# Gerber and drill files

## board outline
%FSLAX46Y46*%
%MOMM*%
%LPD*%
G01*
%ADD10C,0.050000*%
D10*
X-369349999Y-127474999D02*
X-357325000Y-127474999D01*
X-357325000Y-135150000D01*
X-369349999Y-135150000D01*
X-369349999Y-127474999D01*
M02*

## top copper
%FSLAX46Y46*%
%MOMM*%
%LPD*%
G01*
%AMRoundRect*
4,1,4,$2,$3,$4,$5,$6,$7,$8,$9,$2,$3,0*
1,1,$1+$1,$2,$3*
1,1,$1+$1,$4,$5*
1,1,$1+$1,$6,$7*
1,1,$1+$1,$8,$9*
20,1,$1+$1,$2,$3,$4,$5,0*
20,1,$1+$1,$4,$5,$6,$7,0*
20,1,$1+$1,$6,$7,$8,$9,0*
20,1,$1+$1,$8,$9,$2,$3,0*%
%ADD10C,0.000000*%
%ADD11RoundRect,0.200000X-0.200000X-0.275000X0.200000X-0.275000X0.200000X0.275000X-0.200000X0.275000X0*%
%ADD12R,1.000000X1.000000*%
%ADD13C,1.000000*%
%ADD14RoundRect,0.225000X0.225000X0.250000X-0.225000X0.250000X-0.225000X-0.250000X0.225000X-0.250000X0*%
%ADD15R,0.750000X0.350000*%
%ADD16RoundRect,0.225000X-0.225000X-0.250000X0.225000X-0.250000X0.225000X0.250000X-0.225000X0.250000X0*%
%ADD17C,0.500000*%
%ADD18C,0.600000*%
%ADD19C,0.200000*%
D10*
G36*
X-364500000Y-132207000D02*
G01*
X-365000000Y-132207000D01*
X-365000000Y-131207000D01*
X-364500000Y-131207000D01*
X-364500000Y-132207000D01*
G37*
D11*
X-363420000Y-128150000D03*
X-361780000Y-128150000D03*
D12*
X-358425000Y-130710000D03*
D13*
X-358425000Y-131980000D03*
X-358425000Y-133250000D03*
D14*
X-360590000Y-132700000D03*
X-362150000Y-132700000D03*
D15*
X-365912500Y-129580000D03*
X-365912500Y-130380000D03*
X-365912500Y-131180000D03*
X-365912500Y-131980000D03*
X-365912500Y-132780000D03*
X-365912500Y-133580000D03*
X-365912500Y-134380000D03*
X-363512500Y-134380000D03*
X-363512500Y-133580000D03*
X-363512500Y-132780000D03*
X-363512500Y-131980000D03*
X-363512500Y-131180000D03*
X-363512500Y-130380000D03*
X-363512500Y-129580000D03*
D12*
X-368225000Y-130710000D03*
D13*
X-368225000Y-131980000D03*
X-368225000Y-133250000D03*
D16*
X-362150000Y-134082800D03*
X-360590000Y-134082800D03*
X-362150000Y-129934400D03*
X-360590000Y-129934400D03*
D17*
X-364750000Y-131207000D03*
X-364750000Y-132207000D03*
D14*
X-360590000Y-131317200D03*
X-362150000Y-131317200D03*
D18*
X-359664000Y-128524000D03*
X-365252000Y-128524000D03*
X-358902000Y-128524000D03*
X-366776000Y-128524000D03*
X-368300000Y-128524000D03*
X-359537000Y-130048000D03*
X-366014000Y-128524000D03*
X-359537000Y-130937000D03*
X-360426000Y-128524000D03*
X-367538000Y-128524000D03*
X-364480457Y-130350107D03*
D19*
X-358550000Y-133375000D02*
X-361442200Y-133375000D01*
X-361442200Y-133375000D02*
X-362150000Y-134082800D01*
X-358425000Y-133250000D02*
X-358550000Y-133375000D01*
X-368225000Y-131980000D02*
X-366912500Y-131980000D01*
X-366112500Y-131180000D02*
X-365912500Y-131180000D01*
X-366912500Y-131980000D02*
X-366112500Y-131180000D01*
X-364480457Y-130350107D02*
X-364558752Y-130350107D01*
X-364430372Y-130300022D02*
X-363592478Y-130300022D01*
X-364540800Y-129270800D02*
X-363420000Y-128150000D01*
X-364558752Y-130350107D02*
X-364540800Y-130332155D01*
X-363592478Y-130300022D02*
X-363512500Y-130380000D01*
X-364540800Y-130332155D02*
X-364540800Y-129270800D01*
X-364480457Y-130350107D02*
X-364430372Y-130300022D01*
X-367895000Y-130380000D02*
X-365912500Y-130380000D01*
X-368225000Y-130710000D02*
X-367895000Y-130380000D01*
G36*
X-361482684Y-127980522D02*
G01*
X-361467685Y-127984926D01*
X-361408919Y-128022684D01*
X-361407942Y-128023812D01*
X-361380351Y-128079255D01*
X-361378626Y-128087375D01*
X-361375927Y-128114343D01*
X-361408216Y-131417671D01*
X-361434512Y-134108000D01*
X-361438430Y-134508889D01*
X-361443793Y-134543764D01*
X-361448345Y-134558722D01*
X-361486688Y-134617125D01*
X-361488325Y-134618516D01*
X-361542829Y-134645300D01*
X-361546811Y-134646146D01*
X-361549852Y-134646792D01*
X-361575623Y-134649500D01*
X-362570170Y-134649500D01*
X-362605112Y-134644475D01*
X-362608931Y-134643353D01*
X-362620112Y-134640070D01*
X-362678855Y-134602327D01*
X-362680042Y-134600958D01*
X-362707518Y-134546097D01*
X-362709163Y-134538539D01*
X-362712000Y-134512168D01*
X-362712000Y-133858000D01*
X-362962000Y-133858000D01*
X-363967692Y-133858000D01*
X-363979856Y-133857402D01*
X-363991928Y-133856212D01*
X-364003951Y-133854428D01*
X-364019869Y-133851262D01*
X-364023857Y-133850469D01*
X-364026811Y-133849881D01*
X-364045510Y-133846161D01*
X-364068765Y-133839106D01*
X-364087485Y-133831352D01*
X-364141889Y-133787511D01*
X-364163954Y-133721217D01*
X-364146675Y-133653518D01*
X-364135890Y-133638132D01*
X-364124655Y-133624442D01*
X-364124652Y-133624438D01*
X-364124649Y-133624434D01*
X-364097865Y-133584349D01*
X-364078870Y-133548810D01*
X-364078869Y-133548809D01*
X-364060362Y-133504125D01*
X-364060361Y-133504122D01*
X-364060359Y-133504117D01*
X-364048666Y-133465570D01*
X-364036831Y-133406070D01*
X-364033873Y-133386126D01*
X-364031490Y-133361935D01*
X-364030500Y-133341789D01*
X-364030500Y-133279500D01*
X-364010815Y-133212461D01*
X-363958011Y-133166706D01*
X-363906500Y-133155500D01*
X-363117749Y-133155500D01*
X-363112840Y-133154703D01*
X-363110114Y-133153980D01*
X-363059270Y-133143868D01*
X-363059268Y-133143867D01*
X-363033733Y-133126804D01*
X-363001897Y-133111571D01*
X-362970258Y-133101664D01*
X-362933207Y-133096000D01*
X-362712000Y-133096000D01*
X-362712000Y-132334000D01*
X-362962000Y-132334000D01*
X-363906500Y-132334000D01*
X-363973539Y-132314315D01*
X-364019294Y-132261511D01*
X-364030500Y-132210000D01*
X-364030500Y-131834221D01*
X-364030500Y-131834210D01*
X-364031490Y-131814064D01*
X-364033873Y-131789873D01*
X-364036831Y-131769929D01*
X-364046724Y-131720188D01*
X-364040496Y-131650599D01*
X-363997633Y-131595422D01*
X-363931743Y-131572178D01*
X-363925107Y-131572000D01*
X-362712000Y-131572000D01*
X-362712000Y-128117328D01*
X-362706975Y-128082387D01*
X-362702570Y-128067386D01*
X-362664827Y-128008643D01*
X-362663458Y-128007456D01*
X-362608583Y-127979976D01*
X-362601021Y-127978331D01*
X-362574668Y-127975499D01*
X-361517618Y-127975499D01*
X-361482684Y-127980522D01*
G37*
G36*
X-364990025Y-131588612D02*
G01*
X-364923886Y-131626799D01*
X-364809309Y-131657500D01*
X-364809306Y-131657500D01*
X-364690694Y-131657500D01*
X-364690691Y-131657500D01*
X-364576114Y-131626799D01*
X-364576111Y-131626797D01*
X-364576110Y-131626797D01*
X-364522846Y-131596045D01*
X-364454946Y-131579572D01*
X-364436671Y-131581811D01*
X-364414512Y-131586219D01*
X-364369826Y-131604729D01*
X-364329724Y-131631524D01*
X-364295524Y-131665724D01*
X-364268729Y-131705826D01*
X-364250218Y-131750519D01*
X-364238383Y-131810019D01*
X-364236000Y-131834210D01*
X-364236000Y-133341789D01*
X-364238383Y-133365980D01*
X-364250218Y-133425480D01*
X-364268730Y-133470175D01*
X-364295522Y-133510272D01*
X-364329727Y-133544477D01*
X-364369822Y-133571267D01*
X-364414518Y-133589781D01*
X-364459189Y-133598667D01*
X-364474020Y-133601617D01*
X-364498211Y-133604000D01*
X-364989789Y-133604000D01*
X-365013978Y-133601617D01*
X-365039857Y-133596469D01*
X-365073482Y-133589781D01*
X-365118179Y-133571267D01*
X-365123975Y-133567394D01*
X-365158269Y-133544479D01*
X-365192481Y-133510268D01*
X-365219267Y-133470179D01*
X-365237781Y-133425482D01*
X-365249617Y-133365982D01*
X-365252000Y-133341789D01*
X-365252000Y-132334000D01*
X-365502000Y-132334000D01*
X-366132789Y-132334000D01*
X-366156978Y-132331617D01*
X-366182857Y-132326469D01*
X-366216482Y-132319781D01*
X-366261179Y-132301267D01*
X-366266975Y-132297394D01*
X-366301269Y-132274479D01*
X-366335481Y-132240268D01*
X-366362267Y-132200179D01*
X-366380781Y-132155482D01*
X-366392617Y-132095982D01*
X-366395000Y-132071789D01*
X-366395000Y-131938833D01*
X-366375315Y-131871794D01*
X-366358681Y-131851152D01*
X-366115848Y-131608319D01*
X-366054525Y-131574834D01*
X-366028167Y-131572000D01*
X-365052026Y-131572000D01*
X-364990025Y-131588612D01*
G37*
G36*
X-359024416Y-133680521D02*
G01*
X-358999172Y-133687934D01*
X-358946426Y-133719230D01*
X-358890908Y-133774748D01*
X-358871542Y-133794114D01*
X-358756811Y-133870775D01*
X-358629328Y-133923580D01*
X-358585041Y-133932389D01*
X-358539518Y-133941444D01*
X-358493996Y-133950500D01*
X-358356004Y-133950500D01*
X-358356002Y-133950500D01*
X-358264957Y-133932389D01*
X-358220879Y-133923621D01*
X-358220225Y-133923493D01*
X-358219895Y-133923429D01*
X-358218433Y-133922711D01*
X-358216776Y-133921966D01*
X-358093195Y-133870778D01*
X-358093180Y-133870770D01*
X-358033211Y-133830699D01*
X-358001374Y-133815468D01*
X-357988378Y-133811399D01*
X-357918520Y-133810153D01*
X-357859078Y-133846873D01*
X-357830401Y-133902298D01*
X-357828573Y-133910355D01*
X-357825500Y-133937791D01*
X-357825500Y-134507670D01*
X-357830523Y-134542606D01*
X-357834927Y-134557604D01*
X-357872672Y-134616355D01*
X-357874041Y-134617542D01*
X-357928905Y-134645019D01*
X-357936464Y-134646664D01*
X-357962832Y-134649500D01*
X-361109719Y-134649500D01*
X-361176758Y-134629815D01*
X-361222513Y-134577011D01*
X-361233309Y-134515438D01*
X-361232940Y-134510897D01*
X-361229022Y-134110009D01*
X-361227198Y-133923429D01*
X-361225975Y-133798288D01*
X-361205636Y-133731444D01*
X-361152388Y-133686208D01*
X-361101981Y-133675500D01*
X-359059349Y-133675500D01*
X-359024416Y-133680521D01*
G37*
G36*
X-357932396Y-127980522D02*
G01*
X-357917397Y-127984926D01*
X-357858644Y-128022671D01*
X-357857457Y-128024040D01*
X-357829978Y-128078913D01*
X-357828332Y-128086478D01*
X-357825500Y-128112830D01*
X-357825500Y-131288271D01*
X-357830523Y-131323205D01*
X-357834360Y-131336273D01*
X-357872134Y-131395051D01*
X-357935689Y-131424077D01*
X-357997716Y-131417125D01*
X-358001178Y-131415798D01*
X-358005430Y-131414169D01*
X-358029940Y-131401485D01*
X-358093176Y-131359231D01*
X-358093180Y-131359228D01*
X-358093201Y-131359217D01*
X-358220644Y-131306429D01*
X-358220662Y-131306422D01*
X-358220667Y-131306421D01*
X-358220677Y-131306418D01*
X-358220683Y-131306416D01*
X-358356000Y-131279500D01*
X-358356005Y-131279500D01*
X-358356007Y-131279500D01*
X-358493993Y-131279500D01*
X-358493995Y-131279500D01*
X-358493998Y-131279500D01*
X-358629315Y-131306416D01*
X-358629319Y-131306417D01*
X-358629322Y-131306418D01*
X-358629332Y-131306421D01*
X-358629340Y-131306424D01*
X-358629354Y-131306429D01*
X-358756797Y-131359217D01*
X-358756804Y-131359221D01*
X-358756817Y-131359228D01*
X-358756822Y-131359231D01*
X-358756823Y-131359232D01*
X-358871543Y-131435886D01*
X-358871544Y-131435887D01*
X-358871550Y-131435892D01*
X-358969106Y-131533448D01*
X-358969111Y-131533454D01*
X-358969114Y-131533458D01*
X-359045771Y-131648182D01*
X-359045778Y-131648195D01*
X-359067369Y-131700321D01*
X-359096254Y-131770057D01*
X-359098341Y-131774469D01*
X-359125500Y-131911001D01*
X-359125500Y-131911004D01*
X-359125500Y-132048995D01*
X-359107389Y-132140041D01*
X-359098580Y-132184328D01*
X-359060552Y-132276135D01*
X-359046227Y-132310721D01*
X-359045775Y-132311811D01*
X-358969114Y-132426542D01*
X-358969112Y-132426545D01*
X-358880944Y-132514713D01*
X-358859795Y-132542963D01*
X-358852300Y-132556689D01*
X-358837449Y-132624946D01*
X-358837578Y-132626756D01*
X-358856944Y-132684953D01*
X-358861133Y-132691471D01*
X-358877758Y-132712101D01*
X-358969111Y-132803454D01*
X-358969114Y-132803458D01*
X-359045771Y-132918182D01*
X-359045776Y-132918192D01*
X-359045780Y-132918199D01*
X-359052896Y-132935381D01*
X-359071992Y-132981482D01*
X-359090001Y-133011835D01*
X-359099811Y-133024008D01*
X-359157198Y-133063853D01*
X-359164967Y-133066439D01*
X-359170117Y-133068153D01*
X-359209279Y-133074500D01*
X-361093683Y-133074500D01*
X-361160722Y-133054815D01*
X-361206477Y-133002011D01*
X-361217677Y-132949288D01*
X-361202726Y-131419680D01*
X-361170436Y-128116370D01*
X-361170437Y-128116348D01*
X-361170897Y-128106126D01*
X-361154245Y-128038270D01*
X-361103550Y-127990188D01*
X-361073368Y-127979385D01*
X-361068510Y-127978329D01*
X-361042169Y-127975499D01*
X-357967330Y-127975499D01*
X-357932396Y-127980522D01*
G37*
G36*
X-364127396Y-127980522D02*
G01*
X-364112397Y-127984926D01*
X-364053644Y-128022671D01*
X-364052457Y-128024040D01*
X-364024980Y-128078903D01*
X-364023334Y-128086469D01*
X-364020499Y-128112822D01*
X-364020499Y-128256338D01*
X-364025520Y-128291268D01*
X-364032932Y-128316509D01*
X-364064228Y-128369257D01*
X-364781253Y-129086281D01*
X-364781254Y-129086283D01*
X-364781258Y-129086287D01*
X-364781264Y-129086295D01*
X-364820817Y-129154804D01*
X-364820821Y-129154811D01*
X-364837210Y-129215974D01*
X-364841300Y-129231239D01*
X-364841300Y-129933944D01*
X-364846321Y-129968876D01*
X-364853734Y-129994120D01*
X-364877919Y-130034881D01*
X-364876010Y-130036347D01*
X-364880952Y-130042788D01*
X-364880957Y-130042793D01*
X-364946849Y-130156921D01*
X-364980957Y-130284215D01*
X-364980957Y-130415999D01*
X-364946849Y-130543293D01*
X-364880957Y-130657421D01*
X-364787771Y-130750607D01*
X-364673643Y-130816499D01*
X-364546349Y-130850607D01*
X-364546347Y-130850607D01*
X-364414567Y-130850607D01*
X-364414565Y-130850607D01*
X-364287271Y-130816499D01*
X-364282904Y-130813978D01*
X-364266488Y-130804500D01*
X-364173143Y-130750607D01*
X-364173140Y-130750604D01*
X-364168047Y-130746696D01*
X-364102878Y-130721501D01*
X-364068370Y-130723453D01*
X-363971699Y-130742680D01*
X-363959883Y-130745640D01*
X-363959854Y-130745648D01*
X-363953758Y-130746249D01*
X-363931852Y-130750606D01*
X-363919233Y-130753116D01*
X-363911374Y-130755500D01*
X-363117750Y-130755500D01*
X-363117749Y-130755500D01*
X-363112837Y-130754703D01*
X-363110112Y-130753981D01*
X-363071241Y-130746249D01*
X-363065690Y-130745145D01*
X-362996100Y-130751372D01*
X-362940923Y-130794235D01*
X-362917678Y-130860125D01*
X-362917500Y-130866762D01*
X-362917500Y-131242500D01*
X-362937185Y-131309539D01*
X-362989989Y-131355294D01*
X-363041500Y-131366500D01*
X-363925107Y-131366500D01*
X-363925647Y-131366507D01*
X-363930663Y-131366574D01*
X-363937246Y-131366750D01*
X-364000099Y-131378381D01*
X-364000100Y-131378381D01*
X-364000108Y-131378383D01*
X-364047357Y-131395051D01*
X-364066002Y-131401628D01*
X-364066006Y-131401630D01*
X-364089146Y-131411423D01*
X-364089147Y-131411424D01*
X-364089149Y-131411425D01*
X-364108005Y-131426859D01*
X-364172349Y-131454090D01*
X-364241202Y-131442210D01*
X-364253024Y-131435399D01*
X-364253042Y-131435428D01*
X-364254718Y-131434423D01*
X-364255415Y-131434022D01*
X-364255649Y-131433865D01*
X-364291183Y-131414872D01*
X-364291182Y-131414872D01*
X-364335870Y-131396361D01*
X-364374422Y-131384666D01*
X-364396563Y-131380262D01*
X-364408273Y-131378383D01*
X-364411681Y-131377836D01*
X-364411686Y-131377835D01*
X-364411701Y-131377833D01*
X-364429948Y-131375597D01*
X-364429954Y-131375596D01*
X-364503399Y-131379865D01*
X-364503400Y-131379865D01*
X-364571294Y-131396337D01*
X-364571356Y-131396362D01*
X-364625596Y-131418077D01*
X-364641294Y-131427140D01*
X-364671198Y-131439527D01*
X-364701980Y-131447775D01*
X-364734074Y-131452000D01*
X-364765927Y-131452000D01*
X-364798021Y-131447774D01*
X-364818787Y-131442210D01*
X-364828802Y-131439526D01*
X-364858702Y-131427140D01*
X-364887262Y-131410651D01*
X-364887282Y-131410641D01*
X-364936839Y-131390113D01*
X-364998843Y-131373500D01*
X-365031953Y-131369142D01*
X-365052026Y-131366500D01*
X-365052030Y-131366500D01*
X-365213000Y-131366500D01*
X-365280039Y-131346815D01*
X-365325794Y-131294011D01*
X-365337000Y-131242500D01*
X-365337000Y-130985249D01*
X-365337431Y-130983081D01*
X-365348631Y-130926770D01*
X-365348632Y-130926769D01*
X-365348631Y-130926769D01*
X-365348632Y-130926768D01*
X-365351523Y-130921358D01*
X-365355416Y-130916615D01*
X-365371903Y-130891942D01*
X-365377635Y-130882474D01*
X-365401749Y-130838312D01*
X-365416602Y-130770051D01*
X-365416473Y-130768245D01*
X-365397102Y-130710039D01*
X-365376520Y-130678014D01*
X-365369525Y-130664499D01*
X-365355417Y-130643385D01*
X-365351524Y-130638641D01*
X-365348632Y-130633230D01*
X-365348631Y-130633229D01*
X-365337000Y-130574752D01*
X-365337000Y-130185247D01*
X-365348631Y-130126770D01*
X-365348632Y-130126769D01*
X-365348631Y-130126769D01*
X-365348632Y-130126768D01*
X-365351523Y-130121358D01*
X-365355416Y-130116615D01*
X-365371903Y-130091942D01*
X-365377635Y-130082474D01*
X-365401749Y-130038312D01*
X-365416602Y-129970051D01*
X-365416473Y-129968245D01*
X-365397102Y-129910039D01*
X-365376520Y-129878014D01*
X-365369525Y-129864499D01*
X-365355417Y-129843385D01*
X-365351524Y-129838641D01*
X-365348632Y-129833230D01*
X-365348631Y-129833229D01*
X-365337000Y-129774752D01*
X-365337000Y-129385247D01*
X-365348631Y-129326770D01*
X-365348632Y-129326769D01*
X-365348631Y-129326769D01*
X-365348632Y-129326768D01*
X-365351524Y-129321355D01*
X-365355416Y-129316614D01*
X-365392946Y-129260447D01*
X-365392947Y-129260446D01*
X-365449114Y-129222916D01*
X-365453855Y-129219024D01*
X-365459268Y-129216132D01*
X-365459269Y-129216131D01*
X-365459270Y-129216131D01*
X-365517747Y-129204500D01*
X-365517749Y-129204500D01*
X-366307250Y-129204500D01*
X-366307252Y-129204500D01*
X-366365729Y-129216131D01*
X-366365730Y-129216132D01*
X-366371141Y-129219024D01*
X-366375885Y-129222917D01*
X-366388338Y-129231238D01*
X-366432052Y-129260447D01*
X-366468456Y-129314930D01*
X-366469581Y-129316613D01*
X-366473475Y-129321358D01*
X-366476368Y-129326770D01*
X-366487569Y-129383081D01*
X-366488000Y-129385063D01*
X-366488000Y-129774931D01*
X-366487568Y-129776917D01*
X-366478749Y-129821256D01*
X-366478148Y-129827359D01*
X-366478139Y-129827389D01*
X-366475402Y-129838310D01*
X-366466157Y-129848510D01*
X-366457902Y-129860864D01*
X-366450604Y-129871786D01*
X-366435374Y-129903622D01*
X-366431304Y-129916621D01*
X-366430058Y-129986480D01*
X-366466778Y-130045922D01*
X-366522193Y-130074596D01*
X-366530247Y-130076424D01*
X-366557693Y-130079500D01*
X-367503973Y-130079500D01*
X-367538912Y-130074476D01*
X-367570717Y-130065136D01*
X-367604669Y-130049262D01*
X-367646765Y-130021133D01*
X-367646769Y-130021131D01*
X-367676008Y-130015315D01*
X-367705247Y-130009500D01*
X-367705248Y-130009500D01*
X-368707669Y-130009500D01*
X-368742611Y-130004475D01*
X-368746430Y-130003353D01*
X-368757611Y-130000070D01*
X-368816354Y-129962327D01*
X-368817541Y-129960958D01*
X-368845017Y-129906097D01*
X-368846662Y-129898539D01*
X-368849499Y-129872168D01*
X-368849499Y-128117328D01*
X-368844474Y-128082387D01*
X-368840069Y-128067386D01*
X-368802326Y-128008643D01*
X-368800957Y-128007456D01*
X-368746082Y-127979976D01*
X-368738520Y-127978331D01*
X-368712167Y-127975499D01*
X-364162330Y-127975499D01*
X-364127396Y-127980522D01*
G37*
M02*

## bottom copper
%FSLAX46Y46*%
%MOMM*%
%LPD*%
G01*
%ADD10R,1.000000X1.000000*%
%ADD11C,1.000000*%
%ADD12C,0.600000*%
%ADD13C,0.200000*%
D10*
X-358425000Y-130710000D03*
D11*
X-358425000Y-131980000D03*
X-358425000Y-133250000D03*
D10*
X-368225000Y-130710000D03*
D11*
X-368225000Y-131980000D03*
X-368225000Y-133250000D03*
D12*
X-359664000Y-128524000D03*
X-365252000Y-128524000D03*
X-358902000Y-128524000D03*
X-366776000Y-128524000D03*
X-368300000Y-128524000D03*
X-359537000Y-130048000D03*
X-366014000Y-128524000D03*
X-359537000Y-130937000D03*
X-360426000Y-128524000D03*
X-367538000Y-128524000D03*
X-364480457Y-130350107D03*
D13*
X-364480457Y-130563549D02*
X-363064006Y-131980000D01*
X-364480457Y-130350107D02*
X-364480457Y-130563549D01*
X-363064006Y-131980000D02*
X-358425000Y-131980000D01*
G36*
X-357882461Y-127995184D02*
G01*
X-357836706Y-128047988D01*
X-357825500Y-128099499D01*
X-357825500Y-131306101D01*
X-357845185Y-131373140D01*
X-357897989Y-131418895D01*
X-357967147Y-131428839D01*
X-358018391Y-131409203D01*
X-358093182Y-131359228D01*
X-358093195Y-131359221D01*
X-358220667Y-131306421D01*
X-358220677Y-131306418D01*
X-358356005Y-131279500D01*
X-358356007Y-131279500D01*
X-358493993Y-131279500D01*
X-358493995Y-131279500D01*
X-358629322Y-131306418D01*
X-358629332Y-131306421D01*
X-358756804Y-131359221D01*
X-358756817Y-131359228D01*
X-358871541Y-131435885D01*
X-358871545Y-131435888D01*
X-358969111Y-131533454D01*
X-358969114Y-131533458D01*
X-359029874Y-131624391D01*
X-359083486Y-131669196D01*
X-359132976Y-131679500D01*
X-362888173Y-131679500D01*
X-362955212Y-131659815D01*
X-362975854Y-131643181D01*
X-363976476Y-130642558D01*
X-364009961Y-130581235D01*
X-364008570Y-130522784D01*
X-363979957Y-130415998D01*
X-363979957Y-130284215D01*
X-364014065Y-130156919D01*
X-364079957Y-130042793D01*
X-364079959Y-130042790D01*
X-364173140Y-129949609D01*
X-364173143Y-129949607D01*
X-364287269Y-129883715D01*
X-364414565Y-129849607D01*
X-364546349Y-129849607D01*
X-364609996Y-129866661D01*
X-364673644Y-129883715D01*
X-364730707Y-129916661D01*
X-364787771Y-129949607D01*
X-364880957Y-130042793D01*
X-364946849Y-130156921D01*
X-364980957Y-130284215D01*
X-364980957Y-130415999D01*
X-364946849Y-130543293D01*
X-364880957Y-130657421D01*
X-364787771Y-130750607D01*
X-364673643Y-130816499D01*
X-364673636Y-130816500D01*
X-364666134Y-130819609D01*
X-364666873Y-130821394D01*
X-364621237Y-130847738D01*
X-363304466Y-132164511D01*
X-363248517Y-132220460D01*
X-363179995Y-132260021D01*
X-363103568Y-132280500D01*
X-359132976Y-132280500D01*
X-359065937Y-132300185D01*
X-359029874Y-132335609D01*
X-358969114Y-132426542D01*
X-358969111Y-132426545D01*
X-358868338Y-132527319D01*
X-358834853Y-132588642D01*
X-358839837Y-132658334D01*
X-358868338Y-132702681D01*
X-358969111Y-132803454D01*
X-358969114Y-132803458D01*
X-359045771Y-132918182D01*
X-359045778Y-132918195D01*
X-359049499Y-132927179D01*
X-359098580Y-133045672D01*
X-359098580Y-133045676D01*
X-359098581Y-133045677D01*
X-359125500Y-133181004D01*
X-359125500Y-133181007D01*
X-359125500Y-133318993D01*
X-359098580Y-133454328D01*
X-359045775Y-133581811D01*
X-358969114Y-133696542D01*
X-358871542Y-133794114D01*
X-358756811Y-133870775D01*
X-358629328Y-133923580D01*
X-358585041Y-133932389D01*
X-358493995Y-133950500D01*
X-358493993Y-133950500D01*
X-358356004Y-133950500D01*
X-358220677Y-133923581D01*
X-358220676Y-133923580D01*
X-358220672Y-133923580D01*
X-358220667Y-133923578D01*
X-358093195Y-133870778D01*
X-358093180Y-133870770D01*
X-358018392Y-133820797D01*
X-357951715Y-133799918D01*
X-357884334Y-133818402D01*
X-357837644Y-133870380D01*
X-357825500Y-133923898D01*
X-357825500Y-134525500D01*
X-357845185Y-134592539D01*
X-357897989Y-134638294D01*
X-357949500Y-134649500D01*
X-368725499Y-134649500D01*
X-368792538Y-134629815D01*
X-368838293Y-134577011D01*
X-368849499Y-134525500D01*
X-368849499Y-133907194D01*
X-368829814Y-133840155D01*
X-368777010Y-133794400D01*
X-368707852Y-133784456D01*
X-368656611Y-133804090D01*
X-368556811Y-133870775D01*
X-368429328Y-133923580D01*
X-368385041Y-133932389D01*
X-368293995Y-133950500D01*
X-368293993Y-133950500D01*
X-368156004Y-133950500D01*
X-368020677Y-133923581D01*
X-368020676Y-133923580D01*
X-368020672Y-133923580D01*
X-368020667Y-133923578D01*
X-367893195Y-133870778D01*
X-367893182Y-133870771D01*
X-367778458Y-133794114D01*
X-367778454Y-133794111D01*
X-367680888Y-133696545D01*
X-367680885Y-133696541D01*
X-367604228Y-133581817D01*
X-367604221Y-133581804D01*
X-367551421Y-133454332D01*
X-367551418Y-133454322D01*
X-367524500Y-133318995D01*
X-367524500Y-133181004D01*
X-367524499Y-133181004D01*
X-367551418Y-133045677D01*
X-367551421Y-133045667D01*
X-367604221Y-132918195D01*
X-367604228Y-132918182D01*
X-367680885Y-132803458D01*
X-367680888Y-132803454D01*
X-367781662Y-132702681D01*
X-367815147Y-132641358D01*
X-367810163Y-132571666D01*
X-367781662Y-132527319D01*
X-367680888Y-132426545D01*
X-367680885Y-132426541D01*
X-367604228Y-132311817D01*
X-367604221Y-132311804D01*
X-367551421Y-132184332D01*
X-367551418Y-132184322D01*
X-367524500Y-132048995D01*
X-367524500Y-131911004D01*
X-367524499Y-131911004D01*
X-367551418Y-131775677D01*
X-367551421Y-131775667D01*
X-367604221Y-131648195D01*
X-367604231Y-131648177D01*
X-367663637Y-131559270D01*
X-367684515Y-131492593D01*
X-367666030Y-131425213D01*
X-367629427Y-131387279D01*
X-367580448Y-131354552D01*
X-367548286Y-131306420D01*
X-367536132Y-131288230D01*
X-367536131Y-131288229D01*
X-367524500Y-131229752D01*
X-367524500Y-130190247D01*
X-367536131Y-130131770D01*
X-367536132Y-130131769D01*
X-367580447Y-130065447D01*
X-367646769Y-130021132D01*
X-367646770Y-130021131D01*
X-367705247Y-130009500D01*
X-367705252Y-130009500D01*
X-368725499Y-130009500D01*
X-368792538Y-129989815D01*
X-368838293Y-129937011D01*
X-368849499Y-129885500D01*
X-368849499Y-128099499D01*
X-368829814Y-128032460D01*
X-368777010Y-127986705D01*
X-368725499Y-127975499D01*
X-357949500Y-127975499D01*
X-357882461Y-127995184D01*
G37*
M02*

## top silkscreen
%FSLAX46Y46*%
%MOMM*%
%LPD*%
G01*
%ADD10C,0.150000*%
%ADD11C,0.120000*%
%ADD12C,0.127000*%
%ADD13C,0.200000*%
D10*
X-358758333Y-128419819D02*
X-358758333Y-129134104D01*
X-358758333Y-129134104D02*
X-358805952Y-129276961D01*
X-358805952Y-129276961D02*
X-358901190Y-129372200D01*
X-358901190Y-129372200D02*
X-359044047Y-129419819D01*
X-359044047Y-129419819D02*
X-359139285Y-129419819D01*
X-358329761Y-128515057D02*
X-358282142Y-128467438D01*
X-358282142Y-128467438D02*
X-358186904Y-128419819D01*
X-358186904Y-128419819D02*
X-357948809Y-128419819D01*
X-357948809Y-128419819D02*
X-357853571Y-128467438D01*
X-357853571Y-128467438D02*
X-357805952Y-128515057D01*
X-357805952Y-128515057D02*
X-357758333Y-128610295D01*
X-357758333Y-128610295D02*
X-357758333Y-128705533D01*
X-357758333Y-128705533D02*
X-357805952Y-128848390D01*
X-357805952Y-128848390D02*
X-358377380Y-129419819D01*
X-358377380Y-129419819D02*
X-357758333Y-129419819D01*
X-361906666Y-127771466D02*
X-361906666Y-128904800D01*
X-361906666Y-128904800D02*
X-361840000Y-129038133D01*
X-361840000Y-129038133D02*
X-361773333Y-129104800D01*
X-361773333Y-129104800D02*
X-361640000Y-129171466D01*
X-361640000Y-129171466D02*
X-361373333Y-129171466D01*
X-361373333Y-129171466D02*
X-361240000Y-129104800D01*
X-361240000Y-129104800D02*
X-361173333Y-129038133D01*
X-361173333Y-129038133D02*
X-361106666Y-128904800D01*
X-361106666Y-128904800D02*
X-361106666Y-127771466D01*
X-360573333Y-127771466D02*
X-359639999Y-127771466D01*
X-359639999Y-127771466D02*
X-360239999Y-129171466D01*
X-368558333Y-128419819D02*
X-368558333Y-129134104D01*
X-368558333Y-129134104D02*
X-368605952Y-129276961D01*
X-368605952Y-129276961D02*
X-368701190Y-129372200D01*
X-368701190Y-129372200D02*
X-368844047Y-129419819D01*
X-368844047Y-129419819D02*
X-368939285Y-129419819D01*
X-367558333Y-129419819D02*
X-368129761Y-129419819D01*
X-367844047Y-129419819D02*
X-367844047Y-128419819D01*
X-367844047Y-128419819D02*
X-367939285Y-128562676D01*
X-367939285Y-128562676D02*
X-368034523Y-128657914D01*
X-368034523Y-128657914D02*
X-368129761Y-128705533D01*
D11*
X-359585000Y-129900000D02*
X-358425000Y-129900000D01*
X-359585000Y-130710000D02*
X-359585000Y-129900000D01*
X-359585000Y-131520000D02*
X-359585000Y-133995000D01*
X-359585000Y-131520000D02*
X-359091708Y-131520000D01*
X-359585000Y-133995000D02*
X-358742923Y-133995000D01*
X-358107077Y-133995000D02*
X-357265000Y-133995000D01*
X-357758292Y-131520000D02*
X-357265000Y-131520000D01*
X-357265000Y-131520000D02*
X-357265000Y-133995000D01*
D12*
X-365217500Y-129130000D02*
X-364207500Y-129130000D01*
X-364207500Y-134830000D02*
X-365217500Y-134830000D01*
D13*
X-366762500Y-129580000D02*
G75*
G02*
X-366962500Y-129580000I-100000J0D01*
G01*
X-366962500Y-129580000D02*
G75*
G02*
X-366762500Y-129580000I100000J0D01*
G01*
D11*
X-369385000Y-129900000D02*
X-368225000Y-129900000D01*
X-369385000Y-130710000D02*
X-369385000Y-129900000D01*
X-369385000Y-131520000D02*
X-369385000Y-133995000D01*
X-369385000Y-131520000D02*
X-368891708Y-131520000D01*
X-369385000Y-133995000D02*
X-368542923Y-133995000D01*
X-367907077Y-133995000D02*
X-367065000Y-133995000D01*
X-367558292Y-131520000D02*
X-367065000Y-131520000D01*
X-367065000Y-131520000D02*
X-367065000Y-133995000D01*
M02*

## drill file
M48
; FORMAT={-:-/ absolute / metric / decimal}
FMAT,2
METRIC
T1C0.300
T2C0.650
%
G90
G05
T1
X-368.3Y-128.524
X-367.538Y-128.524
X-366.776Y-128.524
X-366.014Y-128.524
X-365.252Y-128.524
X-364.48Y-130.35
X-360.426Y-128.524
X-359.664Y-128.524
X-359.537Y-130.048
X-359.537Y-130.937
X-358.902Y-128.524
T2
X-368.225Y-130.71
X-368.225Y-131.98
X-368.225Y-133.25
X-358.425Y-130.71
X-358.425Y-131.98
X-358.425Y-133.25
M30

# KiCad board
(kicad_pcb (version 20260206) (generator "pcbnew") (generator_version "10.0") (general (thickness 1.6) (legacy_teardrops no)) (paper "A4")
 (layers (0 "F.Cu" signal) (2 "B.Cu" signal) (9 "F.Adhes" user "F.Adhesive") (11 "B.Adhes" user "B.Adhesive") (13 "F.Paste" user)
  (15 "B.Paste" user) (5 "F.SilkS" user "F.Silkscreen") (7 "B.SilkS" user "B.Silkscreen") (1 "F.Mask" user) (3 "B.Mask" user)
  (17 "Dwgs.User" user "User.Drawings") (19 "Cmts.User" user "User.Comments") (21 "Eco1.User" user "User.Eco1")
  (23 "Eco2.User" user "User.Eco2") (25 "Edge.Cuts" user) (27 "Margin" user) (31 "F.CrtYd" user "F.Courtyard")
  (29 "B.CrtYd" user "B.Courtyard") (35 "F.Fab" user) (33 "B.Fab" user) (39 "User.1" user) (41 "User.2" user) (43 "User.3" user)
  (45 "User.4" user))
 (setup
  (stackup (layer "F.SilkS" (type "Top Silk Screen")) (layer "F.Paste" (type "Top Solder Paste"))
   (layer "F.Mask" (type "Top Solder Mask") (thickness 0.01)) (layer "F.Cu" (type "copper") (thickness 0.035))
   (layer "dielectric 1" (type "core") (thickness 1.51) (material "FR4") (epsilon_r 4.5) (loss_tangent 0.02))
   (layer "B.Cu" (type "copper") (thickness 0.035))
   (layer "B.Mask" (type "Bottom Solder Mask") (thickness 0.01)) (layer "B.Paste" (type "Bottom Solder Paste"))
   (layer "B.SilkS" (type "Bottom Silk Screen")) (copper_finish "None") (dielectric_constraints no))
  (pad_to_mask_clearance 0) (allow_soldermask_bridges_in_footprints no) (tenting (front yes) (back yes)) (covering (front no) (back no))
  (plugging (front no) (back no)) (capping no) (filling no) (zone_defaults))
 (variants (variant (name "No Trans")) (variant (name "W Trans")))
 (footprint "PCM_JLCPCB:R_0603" (layer "F.Cu") (at -362.6 128.15)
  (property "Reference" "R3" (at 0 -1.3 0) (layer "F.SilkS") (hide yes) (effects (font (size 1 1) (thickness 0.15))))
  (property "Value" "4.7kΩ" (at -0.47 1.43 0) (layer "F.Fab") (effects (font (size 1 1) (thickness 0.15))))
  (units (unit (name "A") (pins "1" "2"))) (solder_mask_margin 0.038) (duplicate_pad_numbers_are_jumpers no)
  (pad "1" smd roundrect (at -0.82 0) (size 0.8 0.95) (layers "F.Cu" "F.Mask" "F.Paste") (roundrect_rratio 0.25) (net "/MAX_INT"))
  (pad "2" smd roundrect (at 0.82 0) (size 0.8 0.95) (layers "F.Cu" "F.Mask" "F.Paste") (roundrect_rratio 0.25) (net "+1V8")))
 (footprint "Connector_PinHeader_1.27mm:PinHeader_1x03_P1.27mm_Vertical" (layer "F.Cu") (at -358.425 130.71)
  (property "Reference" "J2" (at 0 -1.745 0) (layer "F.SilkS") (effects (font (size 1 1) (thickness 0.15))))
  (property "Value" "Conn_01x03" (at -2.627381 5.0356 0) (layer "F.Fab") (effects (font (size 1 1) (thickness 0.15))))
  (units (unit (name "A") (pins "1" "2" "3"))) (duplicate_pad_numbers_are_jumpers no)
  (fp_line (start -1.16 -0.81) (end 0 -0.81) (stroke (width 0.12) (type solid)) (layer "F.SilkS"))
  (fp_line (start -1.16 0) (end -1.16 -0.81) (stroke (width 0.12) (type solid)) (layer "F.SilkS"))
  (fp_line (start -1.16 0.81) (end -1.16 3.285) (stroke (width 0.12) (type solid)) (layer "F.SilkS"))
  (fp_line (start -1.16 0.81) (end -0.666708 0.81) (stroke (width 0.12) (type solid)) (layer "F.SilkS"))
  (fp_line (start -1.16 3.285) (end -0.317923 3.285) (stroke (width 0.12) (type solid)) (layer "F.SilkS"))
  (fp_line (start 0.317923 3.285) (end 1.16 3.285) (stroke (width 0.12) (type solid)) (layer "F.SilkS"))
  (fp_line (start 0.666708 0.81) (end 1.16 0.81) (stroke (width 0.12) (type solid)) (layer "F.SilkS"))
  (fp_line (start 1.16 0.81) (end 1.16 3.285) (stroke (width 0.12) (type solid)) (layer "F.SilkS"))
  (pad "1" thru_hole rect (at 0 0) (size 1 1) (drill 0.65) (layers "*.Cu" "*.Mask") (remove_unused_layers no) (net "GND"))
  (pad "2" thru_hole circle (at 0 1.27) (size 1 1) (drill 0.65) (layers "*.Cu" "*.Mask") (remove_unused_layers no) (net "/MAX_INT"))
  (pad "3" thru_hole circle (at 0 2.54) (size 1 1) (drill 0.65) (layers "*.Cu" "*.Mask") (remove_unused_layers no) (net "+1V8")))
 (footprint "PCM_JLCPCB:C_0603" (layer "F.Cu") (at -361.37 132.7 180)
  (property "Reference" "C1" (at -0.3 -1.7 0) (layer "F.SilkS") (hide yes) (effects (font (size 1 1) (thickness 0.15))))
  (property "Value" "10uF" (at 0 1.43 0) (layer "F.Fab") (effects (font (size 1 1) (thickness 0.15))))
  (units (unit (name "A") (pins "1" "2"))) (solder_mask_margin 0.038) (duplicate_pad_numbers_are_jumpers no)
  (pad "1" smd roundrect (at -0.78 0 180) (size 0.9 0.95) (layers "F.Cu" "F.Mask" "F.Paste") (roundrect_rratio 0.25) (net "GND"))
  (pad "2" smd roundrect (at 0.78 0 180) (size 0.9 0.95) (layers "F.Cu" "F.Mask" "F.Paste") (roundrect_rratio 0.25) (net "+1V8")))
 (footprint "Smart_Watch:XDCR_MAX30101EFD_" (layer "F.Cu") (at -364.7125 131.98)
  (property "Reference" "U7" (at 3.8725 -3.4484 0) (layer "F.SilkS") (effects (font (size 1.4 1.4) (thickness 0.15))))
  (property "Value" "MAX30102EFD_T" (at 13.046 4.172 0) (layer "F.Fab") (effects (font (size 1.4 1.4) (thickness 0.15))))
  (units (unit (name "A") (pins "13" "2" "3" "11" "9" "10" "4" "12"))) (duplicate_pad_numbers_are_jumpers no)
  (fp_line (start -0.505 -2.85) (end 0.505 -2.85) (stroke (width 0.127) (type solid)) (layer "F.SilkS"))
  (fp_line (start 0.505 2.85) (end -0.505 2.85) (stroke (width 0.127) (type solid)) (layer "F.SilkS"))
  (fp_circle (center -2.15 -2.4) (end -2.05 -2.4) (stroke (width 0.2) (type solid)) (fill no) (layer "F.SilkS"))
  (pad "1" smd rect (at -1.2 -2.4) (size 0.75 0.35) (layers "F.Cu" "F.Mask" "F.Paste") (solder_mask_margin 0.102))
  (pad "2" smd rect (at -1.2 -1.6) (size 0.75 0.35) (layers "F.Cu" "F.Mask" "F.Paste") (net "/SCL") (solder_mask_margin 0.102))
  (pad "3" smd rect (at -1.2 -0.8) (size 0.75 0.35) (layers "F.Cu" "F.Mask" "F.Paste") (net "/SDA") (solder_mask_margin 0.102))
  (pad "4" smd rect (at -1.2 0) (size 0.75 0.35) (layers "F.Cu" "F.Mask" "F.Paste") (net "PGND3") (solder_mask_margin 0.102))
  (pad "5" smd rect (at -1.2 0.8) (size 0.75 0.35) (layers "F.Cu" "F.Mask" "F.Paste") (solder_mask_margin 0.102))
  (pad "6" smd rect (at -1.2 1.6) (size 0.75 0.35) (layers "F.Cu" "F.Mask" "F.Paste") (solder_mask_margin 0.102))
  (pad "7" smd rect (at -1.2 2.4) (size 0.75 0.35) (layers "F.Cu" "F.Mask" "F.Paste") (solder_mask_margin 0.102))
  (pad "8" smd rect (at 1.2 2.4) (size 0.75 0.35) (layers "F.Cu" "F.Mask" "F.Paste") (solder_mask_margin 0.102))
  (pad "9" smd rect (at 1.2 1.6) (size 0.75 0.35) (layers "F.Cu" "F.Mask" "F.Paste") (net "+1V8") (solder_mask_margin 0.102))
  (pad "10" smd rect (at 1.2 0.8) (size 0.75 0.35) (layers "F.Cu" "F.Mask" "F.Paste") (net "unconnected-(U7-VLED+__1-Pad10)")
   (solder_mask_margin 0.102))
  (pad "11" smd rect (at 1.2 0) (size 0.75 0.35) (layers "F.Cu" "F.Mask" "F.Paste") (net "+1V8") (solder_mask_margin 0.102))
  (pad "12" smd rect (at 1.2 -0.8) (size 0.75 0.35) (layers "F.Cu" "F.Mask" "F.Paste") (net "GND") (solder_mask_margin 0.102))
  (pad "13" smd rect (at 1.2 -1.6) (size 0.75 0.35) (layers "F.Cu" "F.Mask" "F.Paste") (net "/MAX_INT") (solder_mask_margin 0.102))
  (pad "14" smd rect (at 1.2 -2.4) (size 0.75 0.35) (layers "F.Cu" "F.Mask" "F.Paste") (solder_mask_margin 0.102)))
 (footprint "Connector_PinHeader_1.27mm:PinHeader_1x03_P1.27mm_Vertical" (layer "F.Cu") (at -368.225 130.71)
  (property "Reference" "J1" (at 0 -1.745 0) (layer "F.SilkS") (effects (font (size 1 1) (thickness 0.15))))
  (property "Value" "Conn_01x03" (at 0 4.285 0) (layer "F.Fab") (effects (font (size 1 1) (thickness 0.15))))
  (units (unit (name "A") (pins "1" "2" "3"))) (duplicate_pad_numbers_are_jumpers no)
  (fp_line (start -1.16 -0.81) (end 0 -0.81) (stroke (width 0.12) (type solid)) (layer "F.SilkS"))
  (fp_line (start -1.16 0) (end -1.16 -0.81) (stroke (width 0.12) (type solid)) (layer "F.SilkS"))
  (fp_line (start -1.16 0.81) (end -1.16 3.285) (stroke (width 0.12) (type solid)) (layer "F.SilkS"))
  (fp_line (start -1.16 0.81) (end -0.666708 0.81) (stroke (width 0.12) (type solid)) (layer "F.SilkS"))
  (fp_line (start -1.16 3.285) (end -0.317923 3.285) (stroke (width 0.12) (type solid)) (layer "F.SilkS"))
  (fp_line (start 0.317923 3.285) (end 1.16 3.285) (stroke (width 0.12) (type solid)) (layer "F.SilkS"))
  (fp_line (start 0.666708 0.81) (end 1.16 0.81) (stroke (width 0.12) (type solid)) (layer "F.SilkS"))
  (fp_line (start 1.16 0.81) (end 1.16 3.285) (stroke (width 0.12) (type solid)) (layer "F.SilkS"))
  (pad "1" thru_hole rect (at 0 0) (size 1 1) (drill 0.65) (layers "*.Cu" "*.Mask") (remove_unused_layers no) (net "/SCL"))
  (pad "2" thru_hole circle (at 0 1.27) (size 1 1) (drill 0.65) (layers "*.Cu" "*.Mask") (remove_unused_layers no) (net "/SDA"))
  (pad "3" thru_hole circle (at 0 2.54) (size 1 1) (drill 0.65) (layers "*.Cu" "*.Mask") (remove_unused_layers no)
   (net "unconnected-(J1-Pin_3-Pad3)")))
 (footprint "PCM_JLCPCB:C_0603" (layer "F.Cu") (at -361.37 134.0828)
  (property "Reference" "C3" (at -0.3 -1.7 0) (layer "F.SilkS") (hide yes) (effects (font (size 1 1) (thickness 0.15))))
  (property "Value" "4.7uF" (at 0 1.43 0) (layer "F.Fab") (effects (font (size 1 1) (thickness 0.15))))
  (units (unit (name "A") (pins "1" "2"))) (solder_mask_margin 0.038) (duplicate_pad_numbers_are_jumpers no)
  (pad "1" smd roundrect (at -0.78 0) (size 0.9 0.95) (layers "F.Cu" "F.Mask" "F.Paste") (roundrect_rratio 0.25) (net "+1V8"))
  (pad "2" smd roundrect (at 0.78 0) (size 0.9 0.95) (layers "F.Cu" "F.Mask" "F.Paste") (roundrect_rratio 0.25) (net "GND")))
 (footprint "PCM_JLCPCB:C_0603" (layer "F.Cu") (at -361.37 129.9344)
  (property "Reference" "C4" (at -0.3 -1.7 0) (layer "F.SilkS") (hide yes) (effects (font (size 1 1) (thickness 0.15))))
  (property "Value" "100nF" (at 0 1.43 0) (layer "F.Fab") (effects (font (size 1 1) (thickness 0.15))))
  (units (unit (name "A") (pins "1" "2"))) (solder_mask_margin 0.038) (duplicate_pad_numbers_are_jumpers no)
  (pad "1" smd roundrect (at -0.78 0) (size 0.9 0.95) (layers "F.Cu" "F.Mask" "F.Paste") (roundrect_rratio 0.25) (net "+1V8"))
  (pad "2" smd roundrect (at 0.78 0) (size 0.9 0.95) (layers "F.Cu" "F.Mask" "F.Paste") (roundrect_rratio 0.25) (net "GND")))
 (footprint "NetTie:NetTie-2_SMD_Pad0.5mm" (layer "F.Cu") (at -364.75 131.707 -90)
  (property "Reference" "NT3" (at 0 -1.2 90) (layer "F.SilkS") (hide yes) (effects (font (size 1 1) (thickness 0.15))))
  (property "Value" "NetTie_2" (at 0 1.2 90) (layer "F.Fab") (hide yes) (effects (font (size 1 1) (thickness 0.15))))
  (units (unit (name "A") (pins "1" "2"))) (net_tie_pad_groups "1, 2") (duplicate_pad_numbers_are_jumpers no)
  (fp_poly (pts (xy -0.5 -0.25) (xy 0.5 -0.25) (xy 0.5 0.25) (xy -0.5 0.25)) (stroke (width 0) (type solid)) (fill yes) (layer "F.Cu"))
  (pad "1" smd circle (at -0.5 0 270) (size 0.5 0.5) (layers "F.Cu") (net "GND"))
  (pad "2" smd circle (at 0.5 0 270) (size 0.5 0.5) (layers "F.Cu") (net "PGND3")))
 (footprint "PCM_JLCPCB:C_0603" (layer "F.Cu") (at -361.37 131.3172 180)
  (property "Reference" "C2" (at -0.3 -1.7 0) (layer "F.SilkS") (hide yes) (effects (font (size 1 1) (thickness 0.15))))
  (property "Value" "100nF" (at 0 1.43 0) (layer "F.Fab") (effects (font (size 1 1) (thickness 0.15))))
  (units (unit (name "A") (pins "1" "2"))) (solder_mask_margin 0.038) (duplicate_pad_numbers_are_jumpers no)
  (pad "1" smd roundrect (at -0.78 0 180) (size 0.9 0.95) (layers "F.Cu" "F.Mask" "F.Paste") (roundrect_rratio 0.25) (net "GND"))
  (pad "2" smd roundrect (at 0.78 0 180) (size 0.9 0.95) (layers "F.Cu" "F.Mask" "F.Paste") (roundrect_rratio 0.25) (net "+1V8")))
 (gr_rect (start -369.349999 127.474999) (end -357.325 135.15) (stroke (width 0.05) (type default)) (fill no) (layer "Edge.Cuts"))
 (via (at -359.664 128.524) (size 0.6) (drill 0.3) (layers "F.Cu" "B.Cu") (free yes) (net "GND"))
 (via (at -365.252 128.524) (size 0.6) (drill 0.3) (layers "F.Cu" "B.Cu") (free yes) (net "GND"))
 (via (at -358.902 128.524) (size 0.6) (drill 0.3) (layers "F.Cu" "B.Cu") (free yes) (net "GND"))
 (via (at -366.776 128.524) (size 0.6) (drill 0.3) (layers "F.Cu" "B.Cu") (free yes) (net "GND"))
 (via (at -368.3 128.524) (size 0.6) (drill 0.3) (layers "F.Cu" "B.Cu") (free yes) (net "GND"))
 (via (at -359.537 130.048) (size 0.6) (drill 0.3) (layers "F.Cu" "B.Cu") (free yes) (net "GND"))
 (via (at -366.014 128.524) (size 0.6) (drill 0.3) (layers "F.Cu" "B.Cu") (free yes) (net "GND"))
 (via (at -359.537 130.937) (size 0.6) (drill 0.3) (layers "F.Cu" "B.Cu") (free yes) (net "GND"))
 (via (at -360.426 128.524) (size 0.6) (drill 0.3) (layers "F.Cu" "B.Cu") (free yes) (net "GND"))
 (via (at -367.538 128.524) (size 0.6) (drill 0.3) (layers "F.Cu" "B.Cu") (free yes) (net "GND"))
 (segment (start -358.55 133.375) (end -361.4422 133.375) (width 0.2) (layer "F.Cu") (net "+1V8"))
 (segment (start -361.4422 133.375) (end -362.15 134.0828) (width 0.2) (layer "F.Cu") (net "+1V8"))
 (segment (start -358.425 133.25) (end -358.55 133.375) (width 0.2) (layer "F.Cu") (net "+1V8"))
 (segment (start -368.225 131.98) (end -366.9125 131.98) (width 0.2) (layer "F.Cu") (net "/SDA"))
 (segment (start -366.1125 131.18) (end -365.9125 131.18) (width 0.2) (layer "F.Cu") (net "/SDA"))
 (segment (start -366.9125 131.98) (end -366.1125 131.18) (width 0.2) (layer "F.Cu") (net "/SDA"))
 (segment (start -364.480457 130.350107) (end -364.558752 130.350107) (width 0.2) (layer "F.Cu") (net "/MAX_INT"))
 (segment (start -364.430372 130.300022) (end -363.592478 130.300022) (width 0.2) (layer "F.Cu") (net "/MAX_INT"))
 (segment (start -364.5408 129.2708) (end -363.42 128.15) (width 0.2) (layer "F.Cu") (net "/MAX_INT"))
 (segment (start -364.558752 130.350107) (end -364.5408 130.332155) (width 0.2) (layer "F.Cu") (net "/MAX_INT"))
 (segment (start -363.592478 130.300022) (end -363.5125 130.38) (width 0.2) (layer "F.Cu") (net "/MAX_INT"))
 (segment (start -364.5408 130.332155) (end -364.5408 129.2708) (width 0.2) (layer "F.Cu") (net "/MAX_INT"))
 (segment (start -364.480457 130.350107) (end -364.430372 130.300022) (width 0.2) (layer "F.Cu") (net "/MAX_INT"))
 (via (at -364.480457 130.350107) (size 0.6) (drill 0.3) (layers "F.Cu" "B.Cu") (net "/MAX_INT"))
 (segment (start -364.480457 130.563549) (end -363.064006 131.98) (width 0.2) (layer "B.Cu") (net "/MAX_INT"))
 (segment (start -364.480457 130.350107) (end -364.480457 130.563549) (width 0.2) (layer "B.Cu") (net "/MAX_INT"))
 (segment (start -363.064006 131.98) (end -358.425 131.98) (width 0.2) (layer "B.Cu") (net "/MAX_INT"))
 (segment (start -367.895 130.38) (end -365.9125 130.38) (width 0.2) (layer "F.Cu") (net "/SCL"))
 (segment (start -368.225 130.71) (end -367.895 130.38) (width 0.2) (layer "F.Cu") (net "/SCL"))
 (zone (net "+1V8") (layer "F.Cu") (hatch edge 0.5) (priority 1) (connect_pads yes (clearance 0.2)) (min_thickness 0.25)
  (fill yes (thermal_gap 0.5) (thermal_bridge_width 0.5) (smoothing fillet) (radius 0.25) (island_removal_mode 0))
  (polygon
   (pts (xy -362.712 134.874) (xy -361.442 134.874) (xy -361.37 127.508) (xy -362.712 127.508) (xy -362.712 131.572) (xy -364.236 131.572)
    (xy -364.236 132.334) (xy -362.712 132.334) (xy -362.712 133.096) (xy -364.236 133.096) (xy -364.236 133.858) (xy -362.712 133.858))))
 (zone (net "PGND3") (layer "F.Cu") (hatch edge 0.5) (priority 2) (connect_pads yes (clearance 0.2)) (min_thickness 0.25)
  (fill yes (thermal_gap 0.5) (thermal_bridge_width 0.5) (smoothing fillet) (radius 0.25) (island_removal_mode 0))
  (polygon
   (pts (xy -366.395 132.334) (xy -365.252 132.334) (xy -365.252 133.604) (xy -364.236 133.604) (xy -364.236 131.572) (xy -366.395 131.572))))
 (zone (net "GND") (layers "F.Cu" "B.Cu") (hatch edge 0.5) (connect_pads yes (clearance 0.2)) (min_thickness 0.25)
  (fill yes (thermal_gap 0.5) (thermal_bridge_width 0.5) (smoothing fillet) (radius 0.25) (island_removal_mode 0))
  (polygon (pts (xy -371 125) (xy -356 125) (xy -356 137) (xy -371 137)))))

